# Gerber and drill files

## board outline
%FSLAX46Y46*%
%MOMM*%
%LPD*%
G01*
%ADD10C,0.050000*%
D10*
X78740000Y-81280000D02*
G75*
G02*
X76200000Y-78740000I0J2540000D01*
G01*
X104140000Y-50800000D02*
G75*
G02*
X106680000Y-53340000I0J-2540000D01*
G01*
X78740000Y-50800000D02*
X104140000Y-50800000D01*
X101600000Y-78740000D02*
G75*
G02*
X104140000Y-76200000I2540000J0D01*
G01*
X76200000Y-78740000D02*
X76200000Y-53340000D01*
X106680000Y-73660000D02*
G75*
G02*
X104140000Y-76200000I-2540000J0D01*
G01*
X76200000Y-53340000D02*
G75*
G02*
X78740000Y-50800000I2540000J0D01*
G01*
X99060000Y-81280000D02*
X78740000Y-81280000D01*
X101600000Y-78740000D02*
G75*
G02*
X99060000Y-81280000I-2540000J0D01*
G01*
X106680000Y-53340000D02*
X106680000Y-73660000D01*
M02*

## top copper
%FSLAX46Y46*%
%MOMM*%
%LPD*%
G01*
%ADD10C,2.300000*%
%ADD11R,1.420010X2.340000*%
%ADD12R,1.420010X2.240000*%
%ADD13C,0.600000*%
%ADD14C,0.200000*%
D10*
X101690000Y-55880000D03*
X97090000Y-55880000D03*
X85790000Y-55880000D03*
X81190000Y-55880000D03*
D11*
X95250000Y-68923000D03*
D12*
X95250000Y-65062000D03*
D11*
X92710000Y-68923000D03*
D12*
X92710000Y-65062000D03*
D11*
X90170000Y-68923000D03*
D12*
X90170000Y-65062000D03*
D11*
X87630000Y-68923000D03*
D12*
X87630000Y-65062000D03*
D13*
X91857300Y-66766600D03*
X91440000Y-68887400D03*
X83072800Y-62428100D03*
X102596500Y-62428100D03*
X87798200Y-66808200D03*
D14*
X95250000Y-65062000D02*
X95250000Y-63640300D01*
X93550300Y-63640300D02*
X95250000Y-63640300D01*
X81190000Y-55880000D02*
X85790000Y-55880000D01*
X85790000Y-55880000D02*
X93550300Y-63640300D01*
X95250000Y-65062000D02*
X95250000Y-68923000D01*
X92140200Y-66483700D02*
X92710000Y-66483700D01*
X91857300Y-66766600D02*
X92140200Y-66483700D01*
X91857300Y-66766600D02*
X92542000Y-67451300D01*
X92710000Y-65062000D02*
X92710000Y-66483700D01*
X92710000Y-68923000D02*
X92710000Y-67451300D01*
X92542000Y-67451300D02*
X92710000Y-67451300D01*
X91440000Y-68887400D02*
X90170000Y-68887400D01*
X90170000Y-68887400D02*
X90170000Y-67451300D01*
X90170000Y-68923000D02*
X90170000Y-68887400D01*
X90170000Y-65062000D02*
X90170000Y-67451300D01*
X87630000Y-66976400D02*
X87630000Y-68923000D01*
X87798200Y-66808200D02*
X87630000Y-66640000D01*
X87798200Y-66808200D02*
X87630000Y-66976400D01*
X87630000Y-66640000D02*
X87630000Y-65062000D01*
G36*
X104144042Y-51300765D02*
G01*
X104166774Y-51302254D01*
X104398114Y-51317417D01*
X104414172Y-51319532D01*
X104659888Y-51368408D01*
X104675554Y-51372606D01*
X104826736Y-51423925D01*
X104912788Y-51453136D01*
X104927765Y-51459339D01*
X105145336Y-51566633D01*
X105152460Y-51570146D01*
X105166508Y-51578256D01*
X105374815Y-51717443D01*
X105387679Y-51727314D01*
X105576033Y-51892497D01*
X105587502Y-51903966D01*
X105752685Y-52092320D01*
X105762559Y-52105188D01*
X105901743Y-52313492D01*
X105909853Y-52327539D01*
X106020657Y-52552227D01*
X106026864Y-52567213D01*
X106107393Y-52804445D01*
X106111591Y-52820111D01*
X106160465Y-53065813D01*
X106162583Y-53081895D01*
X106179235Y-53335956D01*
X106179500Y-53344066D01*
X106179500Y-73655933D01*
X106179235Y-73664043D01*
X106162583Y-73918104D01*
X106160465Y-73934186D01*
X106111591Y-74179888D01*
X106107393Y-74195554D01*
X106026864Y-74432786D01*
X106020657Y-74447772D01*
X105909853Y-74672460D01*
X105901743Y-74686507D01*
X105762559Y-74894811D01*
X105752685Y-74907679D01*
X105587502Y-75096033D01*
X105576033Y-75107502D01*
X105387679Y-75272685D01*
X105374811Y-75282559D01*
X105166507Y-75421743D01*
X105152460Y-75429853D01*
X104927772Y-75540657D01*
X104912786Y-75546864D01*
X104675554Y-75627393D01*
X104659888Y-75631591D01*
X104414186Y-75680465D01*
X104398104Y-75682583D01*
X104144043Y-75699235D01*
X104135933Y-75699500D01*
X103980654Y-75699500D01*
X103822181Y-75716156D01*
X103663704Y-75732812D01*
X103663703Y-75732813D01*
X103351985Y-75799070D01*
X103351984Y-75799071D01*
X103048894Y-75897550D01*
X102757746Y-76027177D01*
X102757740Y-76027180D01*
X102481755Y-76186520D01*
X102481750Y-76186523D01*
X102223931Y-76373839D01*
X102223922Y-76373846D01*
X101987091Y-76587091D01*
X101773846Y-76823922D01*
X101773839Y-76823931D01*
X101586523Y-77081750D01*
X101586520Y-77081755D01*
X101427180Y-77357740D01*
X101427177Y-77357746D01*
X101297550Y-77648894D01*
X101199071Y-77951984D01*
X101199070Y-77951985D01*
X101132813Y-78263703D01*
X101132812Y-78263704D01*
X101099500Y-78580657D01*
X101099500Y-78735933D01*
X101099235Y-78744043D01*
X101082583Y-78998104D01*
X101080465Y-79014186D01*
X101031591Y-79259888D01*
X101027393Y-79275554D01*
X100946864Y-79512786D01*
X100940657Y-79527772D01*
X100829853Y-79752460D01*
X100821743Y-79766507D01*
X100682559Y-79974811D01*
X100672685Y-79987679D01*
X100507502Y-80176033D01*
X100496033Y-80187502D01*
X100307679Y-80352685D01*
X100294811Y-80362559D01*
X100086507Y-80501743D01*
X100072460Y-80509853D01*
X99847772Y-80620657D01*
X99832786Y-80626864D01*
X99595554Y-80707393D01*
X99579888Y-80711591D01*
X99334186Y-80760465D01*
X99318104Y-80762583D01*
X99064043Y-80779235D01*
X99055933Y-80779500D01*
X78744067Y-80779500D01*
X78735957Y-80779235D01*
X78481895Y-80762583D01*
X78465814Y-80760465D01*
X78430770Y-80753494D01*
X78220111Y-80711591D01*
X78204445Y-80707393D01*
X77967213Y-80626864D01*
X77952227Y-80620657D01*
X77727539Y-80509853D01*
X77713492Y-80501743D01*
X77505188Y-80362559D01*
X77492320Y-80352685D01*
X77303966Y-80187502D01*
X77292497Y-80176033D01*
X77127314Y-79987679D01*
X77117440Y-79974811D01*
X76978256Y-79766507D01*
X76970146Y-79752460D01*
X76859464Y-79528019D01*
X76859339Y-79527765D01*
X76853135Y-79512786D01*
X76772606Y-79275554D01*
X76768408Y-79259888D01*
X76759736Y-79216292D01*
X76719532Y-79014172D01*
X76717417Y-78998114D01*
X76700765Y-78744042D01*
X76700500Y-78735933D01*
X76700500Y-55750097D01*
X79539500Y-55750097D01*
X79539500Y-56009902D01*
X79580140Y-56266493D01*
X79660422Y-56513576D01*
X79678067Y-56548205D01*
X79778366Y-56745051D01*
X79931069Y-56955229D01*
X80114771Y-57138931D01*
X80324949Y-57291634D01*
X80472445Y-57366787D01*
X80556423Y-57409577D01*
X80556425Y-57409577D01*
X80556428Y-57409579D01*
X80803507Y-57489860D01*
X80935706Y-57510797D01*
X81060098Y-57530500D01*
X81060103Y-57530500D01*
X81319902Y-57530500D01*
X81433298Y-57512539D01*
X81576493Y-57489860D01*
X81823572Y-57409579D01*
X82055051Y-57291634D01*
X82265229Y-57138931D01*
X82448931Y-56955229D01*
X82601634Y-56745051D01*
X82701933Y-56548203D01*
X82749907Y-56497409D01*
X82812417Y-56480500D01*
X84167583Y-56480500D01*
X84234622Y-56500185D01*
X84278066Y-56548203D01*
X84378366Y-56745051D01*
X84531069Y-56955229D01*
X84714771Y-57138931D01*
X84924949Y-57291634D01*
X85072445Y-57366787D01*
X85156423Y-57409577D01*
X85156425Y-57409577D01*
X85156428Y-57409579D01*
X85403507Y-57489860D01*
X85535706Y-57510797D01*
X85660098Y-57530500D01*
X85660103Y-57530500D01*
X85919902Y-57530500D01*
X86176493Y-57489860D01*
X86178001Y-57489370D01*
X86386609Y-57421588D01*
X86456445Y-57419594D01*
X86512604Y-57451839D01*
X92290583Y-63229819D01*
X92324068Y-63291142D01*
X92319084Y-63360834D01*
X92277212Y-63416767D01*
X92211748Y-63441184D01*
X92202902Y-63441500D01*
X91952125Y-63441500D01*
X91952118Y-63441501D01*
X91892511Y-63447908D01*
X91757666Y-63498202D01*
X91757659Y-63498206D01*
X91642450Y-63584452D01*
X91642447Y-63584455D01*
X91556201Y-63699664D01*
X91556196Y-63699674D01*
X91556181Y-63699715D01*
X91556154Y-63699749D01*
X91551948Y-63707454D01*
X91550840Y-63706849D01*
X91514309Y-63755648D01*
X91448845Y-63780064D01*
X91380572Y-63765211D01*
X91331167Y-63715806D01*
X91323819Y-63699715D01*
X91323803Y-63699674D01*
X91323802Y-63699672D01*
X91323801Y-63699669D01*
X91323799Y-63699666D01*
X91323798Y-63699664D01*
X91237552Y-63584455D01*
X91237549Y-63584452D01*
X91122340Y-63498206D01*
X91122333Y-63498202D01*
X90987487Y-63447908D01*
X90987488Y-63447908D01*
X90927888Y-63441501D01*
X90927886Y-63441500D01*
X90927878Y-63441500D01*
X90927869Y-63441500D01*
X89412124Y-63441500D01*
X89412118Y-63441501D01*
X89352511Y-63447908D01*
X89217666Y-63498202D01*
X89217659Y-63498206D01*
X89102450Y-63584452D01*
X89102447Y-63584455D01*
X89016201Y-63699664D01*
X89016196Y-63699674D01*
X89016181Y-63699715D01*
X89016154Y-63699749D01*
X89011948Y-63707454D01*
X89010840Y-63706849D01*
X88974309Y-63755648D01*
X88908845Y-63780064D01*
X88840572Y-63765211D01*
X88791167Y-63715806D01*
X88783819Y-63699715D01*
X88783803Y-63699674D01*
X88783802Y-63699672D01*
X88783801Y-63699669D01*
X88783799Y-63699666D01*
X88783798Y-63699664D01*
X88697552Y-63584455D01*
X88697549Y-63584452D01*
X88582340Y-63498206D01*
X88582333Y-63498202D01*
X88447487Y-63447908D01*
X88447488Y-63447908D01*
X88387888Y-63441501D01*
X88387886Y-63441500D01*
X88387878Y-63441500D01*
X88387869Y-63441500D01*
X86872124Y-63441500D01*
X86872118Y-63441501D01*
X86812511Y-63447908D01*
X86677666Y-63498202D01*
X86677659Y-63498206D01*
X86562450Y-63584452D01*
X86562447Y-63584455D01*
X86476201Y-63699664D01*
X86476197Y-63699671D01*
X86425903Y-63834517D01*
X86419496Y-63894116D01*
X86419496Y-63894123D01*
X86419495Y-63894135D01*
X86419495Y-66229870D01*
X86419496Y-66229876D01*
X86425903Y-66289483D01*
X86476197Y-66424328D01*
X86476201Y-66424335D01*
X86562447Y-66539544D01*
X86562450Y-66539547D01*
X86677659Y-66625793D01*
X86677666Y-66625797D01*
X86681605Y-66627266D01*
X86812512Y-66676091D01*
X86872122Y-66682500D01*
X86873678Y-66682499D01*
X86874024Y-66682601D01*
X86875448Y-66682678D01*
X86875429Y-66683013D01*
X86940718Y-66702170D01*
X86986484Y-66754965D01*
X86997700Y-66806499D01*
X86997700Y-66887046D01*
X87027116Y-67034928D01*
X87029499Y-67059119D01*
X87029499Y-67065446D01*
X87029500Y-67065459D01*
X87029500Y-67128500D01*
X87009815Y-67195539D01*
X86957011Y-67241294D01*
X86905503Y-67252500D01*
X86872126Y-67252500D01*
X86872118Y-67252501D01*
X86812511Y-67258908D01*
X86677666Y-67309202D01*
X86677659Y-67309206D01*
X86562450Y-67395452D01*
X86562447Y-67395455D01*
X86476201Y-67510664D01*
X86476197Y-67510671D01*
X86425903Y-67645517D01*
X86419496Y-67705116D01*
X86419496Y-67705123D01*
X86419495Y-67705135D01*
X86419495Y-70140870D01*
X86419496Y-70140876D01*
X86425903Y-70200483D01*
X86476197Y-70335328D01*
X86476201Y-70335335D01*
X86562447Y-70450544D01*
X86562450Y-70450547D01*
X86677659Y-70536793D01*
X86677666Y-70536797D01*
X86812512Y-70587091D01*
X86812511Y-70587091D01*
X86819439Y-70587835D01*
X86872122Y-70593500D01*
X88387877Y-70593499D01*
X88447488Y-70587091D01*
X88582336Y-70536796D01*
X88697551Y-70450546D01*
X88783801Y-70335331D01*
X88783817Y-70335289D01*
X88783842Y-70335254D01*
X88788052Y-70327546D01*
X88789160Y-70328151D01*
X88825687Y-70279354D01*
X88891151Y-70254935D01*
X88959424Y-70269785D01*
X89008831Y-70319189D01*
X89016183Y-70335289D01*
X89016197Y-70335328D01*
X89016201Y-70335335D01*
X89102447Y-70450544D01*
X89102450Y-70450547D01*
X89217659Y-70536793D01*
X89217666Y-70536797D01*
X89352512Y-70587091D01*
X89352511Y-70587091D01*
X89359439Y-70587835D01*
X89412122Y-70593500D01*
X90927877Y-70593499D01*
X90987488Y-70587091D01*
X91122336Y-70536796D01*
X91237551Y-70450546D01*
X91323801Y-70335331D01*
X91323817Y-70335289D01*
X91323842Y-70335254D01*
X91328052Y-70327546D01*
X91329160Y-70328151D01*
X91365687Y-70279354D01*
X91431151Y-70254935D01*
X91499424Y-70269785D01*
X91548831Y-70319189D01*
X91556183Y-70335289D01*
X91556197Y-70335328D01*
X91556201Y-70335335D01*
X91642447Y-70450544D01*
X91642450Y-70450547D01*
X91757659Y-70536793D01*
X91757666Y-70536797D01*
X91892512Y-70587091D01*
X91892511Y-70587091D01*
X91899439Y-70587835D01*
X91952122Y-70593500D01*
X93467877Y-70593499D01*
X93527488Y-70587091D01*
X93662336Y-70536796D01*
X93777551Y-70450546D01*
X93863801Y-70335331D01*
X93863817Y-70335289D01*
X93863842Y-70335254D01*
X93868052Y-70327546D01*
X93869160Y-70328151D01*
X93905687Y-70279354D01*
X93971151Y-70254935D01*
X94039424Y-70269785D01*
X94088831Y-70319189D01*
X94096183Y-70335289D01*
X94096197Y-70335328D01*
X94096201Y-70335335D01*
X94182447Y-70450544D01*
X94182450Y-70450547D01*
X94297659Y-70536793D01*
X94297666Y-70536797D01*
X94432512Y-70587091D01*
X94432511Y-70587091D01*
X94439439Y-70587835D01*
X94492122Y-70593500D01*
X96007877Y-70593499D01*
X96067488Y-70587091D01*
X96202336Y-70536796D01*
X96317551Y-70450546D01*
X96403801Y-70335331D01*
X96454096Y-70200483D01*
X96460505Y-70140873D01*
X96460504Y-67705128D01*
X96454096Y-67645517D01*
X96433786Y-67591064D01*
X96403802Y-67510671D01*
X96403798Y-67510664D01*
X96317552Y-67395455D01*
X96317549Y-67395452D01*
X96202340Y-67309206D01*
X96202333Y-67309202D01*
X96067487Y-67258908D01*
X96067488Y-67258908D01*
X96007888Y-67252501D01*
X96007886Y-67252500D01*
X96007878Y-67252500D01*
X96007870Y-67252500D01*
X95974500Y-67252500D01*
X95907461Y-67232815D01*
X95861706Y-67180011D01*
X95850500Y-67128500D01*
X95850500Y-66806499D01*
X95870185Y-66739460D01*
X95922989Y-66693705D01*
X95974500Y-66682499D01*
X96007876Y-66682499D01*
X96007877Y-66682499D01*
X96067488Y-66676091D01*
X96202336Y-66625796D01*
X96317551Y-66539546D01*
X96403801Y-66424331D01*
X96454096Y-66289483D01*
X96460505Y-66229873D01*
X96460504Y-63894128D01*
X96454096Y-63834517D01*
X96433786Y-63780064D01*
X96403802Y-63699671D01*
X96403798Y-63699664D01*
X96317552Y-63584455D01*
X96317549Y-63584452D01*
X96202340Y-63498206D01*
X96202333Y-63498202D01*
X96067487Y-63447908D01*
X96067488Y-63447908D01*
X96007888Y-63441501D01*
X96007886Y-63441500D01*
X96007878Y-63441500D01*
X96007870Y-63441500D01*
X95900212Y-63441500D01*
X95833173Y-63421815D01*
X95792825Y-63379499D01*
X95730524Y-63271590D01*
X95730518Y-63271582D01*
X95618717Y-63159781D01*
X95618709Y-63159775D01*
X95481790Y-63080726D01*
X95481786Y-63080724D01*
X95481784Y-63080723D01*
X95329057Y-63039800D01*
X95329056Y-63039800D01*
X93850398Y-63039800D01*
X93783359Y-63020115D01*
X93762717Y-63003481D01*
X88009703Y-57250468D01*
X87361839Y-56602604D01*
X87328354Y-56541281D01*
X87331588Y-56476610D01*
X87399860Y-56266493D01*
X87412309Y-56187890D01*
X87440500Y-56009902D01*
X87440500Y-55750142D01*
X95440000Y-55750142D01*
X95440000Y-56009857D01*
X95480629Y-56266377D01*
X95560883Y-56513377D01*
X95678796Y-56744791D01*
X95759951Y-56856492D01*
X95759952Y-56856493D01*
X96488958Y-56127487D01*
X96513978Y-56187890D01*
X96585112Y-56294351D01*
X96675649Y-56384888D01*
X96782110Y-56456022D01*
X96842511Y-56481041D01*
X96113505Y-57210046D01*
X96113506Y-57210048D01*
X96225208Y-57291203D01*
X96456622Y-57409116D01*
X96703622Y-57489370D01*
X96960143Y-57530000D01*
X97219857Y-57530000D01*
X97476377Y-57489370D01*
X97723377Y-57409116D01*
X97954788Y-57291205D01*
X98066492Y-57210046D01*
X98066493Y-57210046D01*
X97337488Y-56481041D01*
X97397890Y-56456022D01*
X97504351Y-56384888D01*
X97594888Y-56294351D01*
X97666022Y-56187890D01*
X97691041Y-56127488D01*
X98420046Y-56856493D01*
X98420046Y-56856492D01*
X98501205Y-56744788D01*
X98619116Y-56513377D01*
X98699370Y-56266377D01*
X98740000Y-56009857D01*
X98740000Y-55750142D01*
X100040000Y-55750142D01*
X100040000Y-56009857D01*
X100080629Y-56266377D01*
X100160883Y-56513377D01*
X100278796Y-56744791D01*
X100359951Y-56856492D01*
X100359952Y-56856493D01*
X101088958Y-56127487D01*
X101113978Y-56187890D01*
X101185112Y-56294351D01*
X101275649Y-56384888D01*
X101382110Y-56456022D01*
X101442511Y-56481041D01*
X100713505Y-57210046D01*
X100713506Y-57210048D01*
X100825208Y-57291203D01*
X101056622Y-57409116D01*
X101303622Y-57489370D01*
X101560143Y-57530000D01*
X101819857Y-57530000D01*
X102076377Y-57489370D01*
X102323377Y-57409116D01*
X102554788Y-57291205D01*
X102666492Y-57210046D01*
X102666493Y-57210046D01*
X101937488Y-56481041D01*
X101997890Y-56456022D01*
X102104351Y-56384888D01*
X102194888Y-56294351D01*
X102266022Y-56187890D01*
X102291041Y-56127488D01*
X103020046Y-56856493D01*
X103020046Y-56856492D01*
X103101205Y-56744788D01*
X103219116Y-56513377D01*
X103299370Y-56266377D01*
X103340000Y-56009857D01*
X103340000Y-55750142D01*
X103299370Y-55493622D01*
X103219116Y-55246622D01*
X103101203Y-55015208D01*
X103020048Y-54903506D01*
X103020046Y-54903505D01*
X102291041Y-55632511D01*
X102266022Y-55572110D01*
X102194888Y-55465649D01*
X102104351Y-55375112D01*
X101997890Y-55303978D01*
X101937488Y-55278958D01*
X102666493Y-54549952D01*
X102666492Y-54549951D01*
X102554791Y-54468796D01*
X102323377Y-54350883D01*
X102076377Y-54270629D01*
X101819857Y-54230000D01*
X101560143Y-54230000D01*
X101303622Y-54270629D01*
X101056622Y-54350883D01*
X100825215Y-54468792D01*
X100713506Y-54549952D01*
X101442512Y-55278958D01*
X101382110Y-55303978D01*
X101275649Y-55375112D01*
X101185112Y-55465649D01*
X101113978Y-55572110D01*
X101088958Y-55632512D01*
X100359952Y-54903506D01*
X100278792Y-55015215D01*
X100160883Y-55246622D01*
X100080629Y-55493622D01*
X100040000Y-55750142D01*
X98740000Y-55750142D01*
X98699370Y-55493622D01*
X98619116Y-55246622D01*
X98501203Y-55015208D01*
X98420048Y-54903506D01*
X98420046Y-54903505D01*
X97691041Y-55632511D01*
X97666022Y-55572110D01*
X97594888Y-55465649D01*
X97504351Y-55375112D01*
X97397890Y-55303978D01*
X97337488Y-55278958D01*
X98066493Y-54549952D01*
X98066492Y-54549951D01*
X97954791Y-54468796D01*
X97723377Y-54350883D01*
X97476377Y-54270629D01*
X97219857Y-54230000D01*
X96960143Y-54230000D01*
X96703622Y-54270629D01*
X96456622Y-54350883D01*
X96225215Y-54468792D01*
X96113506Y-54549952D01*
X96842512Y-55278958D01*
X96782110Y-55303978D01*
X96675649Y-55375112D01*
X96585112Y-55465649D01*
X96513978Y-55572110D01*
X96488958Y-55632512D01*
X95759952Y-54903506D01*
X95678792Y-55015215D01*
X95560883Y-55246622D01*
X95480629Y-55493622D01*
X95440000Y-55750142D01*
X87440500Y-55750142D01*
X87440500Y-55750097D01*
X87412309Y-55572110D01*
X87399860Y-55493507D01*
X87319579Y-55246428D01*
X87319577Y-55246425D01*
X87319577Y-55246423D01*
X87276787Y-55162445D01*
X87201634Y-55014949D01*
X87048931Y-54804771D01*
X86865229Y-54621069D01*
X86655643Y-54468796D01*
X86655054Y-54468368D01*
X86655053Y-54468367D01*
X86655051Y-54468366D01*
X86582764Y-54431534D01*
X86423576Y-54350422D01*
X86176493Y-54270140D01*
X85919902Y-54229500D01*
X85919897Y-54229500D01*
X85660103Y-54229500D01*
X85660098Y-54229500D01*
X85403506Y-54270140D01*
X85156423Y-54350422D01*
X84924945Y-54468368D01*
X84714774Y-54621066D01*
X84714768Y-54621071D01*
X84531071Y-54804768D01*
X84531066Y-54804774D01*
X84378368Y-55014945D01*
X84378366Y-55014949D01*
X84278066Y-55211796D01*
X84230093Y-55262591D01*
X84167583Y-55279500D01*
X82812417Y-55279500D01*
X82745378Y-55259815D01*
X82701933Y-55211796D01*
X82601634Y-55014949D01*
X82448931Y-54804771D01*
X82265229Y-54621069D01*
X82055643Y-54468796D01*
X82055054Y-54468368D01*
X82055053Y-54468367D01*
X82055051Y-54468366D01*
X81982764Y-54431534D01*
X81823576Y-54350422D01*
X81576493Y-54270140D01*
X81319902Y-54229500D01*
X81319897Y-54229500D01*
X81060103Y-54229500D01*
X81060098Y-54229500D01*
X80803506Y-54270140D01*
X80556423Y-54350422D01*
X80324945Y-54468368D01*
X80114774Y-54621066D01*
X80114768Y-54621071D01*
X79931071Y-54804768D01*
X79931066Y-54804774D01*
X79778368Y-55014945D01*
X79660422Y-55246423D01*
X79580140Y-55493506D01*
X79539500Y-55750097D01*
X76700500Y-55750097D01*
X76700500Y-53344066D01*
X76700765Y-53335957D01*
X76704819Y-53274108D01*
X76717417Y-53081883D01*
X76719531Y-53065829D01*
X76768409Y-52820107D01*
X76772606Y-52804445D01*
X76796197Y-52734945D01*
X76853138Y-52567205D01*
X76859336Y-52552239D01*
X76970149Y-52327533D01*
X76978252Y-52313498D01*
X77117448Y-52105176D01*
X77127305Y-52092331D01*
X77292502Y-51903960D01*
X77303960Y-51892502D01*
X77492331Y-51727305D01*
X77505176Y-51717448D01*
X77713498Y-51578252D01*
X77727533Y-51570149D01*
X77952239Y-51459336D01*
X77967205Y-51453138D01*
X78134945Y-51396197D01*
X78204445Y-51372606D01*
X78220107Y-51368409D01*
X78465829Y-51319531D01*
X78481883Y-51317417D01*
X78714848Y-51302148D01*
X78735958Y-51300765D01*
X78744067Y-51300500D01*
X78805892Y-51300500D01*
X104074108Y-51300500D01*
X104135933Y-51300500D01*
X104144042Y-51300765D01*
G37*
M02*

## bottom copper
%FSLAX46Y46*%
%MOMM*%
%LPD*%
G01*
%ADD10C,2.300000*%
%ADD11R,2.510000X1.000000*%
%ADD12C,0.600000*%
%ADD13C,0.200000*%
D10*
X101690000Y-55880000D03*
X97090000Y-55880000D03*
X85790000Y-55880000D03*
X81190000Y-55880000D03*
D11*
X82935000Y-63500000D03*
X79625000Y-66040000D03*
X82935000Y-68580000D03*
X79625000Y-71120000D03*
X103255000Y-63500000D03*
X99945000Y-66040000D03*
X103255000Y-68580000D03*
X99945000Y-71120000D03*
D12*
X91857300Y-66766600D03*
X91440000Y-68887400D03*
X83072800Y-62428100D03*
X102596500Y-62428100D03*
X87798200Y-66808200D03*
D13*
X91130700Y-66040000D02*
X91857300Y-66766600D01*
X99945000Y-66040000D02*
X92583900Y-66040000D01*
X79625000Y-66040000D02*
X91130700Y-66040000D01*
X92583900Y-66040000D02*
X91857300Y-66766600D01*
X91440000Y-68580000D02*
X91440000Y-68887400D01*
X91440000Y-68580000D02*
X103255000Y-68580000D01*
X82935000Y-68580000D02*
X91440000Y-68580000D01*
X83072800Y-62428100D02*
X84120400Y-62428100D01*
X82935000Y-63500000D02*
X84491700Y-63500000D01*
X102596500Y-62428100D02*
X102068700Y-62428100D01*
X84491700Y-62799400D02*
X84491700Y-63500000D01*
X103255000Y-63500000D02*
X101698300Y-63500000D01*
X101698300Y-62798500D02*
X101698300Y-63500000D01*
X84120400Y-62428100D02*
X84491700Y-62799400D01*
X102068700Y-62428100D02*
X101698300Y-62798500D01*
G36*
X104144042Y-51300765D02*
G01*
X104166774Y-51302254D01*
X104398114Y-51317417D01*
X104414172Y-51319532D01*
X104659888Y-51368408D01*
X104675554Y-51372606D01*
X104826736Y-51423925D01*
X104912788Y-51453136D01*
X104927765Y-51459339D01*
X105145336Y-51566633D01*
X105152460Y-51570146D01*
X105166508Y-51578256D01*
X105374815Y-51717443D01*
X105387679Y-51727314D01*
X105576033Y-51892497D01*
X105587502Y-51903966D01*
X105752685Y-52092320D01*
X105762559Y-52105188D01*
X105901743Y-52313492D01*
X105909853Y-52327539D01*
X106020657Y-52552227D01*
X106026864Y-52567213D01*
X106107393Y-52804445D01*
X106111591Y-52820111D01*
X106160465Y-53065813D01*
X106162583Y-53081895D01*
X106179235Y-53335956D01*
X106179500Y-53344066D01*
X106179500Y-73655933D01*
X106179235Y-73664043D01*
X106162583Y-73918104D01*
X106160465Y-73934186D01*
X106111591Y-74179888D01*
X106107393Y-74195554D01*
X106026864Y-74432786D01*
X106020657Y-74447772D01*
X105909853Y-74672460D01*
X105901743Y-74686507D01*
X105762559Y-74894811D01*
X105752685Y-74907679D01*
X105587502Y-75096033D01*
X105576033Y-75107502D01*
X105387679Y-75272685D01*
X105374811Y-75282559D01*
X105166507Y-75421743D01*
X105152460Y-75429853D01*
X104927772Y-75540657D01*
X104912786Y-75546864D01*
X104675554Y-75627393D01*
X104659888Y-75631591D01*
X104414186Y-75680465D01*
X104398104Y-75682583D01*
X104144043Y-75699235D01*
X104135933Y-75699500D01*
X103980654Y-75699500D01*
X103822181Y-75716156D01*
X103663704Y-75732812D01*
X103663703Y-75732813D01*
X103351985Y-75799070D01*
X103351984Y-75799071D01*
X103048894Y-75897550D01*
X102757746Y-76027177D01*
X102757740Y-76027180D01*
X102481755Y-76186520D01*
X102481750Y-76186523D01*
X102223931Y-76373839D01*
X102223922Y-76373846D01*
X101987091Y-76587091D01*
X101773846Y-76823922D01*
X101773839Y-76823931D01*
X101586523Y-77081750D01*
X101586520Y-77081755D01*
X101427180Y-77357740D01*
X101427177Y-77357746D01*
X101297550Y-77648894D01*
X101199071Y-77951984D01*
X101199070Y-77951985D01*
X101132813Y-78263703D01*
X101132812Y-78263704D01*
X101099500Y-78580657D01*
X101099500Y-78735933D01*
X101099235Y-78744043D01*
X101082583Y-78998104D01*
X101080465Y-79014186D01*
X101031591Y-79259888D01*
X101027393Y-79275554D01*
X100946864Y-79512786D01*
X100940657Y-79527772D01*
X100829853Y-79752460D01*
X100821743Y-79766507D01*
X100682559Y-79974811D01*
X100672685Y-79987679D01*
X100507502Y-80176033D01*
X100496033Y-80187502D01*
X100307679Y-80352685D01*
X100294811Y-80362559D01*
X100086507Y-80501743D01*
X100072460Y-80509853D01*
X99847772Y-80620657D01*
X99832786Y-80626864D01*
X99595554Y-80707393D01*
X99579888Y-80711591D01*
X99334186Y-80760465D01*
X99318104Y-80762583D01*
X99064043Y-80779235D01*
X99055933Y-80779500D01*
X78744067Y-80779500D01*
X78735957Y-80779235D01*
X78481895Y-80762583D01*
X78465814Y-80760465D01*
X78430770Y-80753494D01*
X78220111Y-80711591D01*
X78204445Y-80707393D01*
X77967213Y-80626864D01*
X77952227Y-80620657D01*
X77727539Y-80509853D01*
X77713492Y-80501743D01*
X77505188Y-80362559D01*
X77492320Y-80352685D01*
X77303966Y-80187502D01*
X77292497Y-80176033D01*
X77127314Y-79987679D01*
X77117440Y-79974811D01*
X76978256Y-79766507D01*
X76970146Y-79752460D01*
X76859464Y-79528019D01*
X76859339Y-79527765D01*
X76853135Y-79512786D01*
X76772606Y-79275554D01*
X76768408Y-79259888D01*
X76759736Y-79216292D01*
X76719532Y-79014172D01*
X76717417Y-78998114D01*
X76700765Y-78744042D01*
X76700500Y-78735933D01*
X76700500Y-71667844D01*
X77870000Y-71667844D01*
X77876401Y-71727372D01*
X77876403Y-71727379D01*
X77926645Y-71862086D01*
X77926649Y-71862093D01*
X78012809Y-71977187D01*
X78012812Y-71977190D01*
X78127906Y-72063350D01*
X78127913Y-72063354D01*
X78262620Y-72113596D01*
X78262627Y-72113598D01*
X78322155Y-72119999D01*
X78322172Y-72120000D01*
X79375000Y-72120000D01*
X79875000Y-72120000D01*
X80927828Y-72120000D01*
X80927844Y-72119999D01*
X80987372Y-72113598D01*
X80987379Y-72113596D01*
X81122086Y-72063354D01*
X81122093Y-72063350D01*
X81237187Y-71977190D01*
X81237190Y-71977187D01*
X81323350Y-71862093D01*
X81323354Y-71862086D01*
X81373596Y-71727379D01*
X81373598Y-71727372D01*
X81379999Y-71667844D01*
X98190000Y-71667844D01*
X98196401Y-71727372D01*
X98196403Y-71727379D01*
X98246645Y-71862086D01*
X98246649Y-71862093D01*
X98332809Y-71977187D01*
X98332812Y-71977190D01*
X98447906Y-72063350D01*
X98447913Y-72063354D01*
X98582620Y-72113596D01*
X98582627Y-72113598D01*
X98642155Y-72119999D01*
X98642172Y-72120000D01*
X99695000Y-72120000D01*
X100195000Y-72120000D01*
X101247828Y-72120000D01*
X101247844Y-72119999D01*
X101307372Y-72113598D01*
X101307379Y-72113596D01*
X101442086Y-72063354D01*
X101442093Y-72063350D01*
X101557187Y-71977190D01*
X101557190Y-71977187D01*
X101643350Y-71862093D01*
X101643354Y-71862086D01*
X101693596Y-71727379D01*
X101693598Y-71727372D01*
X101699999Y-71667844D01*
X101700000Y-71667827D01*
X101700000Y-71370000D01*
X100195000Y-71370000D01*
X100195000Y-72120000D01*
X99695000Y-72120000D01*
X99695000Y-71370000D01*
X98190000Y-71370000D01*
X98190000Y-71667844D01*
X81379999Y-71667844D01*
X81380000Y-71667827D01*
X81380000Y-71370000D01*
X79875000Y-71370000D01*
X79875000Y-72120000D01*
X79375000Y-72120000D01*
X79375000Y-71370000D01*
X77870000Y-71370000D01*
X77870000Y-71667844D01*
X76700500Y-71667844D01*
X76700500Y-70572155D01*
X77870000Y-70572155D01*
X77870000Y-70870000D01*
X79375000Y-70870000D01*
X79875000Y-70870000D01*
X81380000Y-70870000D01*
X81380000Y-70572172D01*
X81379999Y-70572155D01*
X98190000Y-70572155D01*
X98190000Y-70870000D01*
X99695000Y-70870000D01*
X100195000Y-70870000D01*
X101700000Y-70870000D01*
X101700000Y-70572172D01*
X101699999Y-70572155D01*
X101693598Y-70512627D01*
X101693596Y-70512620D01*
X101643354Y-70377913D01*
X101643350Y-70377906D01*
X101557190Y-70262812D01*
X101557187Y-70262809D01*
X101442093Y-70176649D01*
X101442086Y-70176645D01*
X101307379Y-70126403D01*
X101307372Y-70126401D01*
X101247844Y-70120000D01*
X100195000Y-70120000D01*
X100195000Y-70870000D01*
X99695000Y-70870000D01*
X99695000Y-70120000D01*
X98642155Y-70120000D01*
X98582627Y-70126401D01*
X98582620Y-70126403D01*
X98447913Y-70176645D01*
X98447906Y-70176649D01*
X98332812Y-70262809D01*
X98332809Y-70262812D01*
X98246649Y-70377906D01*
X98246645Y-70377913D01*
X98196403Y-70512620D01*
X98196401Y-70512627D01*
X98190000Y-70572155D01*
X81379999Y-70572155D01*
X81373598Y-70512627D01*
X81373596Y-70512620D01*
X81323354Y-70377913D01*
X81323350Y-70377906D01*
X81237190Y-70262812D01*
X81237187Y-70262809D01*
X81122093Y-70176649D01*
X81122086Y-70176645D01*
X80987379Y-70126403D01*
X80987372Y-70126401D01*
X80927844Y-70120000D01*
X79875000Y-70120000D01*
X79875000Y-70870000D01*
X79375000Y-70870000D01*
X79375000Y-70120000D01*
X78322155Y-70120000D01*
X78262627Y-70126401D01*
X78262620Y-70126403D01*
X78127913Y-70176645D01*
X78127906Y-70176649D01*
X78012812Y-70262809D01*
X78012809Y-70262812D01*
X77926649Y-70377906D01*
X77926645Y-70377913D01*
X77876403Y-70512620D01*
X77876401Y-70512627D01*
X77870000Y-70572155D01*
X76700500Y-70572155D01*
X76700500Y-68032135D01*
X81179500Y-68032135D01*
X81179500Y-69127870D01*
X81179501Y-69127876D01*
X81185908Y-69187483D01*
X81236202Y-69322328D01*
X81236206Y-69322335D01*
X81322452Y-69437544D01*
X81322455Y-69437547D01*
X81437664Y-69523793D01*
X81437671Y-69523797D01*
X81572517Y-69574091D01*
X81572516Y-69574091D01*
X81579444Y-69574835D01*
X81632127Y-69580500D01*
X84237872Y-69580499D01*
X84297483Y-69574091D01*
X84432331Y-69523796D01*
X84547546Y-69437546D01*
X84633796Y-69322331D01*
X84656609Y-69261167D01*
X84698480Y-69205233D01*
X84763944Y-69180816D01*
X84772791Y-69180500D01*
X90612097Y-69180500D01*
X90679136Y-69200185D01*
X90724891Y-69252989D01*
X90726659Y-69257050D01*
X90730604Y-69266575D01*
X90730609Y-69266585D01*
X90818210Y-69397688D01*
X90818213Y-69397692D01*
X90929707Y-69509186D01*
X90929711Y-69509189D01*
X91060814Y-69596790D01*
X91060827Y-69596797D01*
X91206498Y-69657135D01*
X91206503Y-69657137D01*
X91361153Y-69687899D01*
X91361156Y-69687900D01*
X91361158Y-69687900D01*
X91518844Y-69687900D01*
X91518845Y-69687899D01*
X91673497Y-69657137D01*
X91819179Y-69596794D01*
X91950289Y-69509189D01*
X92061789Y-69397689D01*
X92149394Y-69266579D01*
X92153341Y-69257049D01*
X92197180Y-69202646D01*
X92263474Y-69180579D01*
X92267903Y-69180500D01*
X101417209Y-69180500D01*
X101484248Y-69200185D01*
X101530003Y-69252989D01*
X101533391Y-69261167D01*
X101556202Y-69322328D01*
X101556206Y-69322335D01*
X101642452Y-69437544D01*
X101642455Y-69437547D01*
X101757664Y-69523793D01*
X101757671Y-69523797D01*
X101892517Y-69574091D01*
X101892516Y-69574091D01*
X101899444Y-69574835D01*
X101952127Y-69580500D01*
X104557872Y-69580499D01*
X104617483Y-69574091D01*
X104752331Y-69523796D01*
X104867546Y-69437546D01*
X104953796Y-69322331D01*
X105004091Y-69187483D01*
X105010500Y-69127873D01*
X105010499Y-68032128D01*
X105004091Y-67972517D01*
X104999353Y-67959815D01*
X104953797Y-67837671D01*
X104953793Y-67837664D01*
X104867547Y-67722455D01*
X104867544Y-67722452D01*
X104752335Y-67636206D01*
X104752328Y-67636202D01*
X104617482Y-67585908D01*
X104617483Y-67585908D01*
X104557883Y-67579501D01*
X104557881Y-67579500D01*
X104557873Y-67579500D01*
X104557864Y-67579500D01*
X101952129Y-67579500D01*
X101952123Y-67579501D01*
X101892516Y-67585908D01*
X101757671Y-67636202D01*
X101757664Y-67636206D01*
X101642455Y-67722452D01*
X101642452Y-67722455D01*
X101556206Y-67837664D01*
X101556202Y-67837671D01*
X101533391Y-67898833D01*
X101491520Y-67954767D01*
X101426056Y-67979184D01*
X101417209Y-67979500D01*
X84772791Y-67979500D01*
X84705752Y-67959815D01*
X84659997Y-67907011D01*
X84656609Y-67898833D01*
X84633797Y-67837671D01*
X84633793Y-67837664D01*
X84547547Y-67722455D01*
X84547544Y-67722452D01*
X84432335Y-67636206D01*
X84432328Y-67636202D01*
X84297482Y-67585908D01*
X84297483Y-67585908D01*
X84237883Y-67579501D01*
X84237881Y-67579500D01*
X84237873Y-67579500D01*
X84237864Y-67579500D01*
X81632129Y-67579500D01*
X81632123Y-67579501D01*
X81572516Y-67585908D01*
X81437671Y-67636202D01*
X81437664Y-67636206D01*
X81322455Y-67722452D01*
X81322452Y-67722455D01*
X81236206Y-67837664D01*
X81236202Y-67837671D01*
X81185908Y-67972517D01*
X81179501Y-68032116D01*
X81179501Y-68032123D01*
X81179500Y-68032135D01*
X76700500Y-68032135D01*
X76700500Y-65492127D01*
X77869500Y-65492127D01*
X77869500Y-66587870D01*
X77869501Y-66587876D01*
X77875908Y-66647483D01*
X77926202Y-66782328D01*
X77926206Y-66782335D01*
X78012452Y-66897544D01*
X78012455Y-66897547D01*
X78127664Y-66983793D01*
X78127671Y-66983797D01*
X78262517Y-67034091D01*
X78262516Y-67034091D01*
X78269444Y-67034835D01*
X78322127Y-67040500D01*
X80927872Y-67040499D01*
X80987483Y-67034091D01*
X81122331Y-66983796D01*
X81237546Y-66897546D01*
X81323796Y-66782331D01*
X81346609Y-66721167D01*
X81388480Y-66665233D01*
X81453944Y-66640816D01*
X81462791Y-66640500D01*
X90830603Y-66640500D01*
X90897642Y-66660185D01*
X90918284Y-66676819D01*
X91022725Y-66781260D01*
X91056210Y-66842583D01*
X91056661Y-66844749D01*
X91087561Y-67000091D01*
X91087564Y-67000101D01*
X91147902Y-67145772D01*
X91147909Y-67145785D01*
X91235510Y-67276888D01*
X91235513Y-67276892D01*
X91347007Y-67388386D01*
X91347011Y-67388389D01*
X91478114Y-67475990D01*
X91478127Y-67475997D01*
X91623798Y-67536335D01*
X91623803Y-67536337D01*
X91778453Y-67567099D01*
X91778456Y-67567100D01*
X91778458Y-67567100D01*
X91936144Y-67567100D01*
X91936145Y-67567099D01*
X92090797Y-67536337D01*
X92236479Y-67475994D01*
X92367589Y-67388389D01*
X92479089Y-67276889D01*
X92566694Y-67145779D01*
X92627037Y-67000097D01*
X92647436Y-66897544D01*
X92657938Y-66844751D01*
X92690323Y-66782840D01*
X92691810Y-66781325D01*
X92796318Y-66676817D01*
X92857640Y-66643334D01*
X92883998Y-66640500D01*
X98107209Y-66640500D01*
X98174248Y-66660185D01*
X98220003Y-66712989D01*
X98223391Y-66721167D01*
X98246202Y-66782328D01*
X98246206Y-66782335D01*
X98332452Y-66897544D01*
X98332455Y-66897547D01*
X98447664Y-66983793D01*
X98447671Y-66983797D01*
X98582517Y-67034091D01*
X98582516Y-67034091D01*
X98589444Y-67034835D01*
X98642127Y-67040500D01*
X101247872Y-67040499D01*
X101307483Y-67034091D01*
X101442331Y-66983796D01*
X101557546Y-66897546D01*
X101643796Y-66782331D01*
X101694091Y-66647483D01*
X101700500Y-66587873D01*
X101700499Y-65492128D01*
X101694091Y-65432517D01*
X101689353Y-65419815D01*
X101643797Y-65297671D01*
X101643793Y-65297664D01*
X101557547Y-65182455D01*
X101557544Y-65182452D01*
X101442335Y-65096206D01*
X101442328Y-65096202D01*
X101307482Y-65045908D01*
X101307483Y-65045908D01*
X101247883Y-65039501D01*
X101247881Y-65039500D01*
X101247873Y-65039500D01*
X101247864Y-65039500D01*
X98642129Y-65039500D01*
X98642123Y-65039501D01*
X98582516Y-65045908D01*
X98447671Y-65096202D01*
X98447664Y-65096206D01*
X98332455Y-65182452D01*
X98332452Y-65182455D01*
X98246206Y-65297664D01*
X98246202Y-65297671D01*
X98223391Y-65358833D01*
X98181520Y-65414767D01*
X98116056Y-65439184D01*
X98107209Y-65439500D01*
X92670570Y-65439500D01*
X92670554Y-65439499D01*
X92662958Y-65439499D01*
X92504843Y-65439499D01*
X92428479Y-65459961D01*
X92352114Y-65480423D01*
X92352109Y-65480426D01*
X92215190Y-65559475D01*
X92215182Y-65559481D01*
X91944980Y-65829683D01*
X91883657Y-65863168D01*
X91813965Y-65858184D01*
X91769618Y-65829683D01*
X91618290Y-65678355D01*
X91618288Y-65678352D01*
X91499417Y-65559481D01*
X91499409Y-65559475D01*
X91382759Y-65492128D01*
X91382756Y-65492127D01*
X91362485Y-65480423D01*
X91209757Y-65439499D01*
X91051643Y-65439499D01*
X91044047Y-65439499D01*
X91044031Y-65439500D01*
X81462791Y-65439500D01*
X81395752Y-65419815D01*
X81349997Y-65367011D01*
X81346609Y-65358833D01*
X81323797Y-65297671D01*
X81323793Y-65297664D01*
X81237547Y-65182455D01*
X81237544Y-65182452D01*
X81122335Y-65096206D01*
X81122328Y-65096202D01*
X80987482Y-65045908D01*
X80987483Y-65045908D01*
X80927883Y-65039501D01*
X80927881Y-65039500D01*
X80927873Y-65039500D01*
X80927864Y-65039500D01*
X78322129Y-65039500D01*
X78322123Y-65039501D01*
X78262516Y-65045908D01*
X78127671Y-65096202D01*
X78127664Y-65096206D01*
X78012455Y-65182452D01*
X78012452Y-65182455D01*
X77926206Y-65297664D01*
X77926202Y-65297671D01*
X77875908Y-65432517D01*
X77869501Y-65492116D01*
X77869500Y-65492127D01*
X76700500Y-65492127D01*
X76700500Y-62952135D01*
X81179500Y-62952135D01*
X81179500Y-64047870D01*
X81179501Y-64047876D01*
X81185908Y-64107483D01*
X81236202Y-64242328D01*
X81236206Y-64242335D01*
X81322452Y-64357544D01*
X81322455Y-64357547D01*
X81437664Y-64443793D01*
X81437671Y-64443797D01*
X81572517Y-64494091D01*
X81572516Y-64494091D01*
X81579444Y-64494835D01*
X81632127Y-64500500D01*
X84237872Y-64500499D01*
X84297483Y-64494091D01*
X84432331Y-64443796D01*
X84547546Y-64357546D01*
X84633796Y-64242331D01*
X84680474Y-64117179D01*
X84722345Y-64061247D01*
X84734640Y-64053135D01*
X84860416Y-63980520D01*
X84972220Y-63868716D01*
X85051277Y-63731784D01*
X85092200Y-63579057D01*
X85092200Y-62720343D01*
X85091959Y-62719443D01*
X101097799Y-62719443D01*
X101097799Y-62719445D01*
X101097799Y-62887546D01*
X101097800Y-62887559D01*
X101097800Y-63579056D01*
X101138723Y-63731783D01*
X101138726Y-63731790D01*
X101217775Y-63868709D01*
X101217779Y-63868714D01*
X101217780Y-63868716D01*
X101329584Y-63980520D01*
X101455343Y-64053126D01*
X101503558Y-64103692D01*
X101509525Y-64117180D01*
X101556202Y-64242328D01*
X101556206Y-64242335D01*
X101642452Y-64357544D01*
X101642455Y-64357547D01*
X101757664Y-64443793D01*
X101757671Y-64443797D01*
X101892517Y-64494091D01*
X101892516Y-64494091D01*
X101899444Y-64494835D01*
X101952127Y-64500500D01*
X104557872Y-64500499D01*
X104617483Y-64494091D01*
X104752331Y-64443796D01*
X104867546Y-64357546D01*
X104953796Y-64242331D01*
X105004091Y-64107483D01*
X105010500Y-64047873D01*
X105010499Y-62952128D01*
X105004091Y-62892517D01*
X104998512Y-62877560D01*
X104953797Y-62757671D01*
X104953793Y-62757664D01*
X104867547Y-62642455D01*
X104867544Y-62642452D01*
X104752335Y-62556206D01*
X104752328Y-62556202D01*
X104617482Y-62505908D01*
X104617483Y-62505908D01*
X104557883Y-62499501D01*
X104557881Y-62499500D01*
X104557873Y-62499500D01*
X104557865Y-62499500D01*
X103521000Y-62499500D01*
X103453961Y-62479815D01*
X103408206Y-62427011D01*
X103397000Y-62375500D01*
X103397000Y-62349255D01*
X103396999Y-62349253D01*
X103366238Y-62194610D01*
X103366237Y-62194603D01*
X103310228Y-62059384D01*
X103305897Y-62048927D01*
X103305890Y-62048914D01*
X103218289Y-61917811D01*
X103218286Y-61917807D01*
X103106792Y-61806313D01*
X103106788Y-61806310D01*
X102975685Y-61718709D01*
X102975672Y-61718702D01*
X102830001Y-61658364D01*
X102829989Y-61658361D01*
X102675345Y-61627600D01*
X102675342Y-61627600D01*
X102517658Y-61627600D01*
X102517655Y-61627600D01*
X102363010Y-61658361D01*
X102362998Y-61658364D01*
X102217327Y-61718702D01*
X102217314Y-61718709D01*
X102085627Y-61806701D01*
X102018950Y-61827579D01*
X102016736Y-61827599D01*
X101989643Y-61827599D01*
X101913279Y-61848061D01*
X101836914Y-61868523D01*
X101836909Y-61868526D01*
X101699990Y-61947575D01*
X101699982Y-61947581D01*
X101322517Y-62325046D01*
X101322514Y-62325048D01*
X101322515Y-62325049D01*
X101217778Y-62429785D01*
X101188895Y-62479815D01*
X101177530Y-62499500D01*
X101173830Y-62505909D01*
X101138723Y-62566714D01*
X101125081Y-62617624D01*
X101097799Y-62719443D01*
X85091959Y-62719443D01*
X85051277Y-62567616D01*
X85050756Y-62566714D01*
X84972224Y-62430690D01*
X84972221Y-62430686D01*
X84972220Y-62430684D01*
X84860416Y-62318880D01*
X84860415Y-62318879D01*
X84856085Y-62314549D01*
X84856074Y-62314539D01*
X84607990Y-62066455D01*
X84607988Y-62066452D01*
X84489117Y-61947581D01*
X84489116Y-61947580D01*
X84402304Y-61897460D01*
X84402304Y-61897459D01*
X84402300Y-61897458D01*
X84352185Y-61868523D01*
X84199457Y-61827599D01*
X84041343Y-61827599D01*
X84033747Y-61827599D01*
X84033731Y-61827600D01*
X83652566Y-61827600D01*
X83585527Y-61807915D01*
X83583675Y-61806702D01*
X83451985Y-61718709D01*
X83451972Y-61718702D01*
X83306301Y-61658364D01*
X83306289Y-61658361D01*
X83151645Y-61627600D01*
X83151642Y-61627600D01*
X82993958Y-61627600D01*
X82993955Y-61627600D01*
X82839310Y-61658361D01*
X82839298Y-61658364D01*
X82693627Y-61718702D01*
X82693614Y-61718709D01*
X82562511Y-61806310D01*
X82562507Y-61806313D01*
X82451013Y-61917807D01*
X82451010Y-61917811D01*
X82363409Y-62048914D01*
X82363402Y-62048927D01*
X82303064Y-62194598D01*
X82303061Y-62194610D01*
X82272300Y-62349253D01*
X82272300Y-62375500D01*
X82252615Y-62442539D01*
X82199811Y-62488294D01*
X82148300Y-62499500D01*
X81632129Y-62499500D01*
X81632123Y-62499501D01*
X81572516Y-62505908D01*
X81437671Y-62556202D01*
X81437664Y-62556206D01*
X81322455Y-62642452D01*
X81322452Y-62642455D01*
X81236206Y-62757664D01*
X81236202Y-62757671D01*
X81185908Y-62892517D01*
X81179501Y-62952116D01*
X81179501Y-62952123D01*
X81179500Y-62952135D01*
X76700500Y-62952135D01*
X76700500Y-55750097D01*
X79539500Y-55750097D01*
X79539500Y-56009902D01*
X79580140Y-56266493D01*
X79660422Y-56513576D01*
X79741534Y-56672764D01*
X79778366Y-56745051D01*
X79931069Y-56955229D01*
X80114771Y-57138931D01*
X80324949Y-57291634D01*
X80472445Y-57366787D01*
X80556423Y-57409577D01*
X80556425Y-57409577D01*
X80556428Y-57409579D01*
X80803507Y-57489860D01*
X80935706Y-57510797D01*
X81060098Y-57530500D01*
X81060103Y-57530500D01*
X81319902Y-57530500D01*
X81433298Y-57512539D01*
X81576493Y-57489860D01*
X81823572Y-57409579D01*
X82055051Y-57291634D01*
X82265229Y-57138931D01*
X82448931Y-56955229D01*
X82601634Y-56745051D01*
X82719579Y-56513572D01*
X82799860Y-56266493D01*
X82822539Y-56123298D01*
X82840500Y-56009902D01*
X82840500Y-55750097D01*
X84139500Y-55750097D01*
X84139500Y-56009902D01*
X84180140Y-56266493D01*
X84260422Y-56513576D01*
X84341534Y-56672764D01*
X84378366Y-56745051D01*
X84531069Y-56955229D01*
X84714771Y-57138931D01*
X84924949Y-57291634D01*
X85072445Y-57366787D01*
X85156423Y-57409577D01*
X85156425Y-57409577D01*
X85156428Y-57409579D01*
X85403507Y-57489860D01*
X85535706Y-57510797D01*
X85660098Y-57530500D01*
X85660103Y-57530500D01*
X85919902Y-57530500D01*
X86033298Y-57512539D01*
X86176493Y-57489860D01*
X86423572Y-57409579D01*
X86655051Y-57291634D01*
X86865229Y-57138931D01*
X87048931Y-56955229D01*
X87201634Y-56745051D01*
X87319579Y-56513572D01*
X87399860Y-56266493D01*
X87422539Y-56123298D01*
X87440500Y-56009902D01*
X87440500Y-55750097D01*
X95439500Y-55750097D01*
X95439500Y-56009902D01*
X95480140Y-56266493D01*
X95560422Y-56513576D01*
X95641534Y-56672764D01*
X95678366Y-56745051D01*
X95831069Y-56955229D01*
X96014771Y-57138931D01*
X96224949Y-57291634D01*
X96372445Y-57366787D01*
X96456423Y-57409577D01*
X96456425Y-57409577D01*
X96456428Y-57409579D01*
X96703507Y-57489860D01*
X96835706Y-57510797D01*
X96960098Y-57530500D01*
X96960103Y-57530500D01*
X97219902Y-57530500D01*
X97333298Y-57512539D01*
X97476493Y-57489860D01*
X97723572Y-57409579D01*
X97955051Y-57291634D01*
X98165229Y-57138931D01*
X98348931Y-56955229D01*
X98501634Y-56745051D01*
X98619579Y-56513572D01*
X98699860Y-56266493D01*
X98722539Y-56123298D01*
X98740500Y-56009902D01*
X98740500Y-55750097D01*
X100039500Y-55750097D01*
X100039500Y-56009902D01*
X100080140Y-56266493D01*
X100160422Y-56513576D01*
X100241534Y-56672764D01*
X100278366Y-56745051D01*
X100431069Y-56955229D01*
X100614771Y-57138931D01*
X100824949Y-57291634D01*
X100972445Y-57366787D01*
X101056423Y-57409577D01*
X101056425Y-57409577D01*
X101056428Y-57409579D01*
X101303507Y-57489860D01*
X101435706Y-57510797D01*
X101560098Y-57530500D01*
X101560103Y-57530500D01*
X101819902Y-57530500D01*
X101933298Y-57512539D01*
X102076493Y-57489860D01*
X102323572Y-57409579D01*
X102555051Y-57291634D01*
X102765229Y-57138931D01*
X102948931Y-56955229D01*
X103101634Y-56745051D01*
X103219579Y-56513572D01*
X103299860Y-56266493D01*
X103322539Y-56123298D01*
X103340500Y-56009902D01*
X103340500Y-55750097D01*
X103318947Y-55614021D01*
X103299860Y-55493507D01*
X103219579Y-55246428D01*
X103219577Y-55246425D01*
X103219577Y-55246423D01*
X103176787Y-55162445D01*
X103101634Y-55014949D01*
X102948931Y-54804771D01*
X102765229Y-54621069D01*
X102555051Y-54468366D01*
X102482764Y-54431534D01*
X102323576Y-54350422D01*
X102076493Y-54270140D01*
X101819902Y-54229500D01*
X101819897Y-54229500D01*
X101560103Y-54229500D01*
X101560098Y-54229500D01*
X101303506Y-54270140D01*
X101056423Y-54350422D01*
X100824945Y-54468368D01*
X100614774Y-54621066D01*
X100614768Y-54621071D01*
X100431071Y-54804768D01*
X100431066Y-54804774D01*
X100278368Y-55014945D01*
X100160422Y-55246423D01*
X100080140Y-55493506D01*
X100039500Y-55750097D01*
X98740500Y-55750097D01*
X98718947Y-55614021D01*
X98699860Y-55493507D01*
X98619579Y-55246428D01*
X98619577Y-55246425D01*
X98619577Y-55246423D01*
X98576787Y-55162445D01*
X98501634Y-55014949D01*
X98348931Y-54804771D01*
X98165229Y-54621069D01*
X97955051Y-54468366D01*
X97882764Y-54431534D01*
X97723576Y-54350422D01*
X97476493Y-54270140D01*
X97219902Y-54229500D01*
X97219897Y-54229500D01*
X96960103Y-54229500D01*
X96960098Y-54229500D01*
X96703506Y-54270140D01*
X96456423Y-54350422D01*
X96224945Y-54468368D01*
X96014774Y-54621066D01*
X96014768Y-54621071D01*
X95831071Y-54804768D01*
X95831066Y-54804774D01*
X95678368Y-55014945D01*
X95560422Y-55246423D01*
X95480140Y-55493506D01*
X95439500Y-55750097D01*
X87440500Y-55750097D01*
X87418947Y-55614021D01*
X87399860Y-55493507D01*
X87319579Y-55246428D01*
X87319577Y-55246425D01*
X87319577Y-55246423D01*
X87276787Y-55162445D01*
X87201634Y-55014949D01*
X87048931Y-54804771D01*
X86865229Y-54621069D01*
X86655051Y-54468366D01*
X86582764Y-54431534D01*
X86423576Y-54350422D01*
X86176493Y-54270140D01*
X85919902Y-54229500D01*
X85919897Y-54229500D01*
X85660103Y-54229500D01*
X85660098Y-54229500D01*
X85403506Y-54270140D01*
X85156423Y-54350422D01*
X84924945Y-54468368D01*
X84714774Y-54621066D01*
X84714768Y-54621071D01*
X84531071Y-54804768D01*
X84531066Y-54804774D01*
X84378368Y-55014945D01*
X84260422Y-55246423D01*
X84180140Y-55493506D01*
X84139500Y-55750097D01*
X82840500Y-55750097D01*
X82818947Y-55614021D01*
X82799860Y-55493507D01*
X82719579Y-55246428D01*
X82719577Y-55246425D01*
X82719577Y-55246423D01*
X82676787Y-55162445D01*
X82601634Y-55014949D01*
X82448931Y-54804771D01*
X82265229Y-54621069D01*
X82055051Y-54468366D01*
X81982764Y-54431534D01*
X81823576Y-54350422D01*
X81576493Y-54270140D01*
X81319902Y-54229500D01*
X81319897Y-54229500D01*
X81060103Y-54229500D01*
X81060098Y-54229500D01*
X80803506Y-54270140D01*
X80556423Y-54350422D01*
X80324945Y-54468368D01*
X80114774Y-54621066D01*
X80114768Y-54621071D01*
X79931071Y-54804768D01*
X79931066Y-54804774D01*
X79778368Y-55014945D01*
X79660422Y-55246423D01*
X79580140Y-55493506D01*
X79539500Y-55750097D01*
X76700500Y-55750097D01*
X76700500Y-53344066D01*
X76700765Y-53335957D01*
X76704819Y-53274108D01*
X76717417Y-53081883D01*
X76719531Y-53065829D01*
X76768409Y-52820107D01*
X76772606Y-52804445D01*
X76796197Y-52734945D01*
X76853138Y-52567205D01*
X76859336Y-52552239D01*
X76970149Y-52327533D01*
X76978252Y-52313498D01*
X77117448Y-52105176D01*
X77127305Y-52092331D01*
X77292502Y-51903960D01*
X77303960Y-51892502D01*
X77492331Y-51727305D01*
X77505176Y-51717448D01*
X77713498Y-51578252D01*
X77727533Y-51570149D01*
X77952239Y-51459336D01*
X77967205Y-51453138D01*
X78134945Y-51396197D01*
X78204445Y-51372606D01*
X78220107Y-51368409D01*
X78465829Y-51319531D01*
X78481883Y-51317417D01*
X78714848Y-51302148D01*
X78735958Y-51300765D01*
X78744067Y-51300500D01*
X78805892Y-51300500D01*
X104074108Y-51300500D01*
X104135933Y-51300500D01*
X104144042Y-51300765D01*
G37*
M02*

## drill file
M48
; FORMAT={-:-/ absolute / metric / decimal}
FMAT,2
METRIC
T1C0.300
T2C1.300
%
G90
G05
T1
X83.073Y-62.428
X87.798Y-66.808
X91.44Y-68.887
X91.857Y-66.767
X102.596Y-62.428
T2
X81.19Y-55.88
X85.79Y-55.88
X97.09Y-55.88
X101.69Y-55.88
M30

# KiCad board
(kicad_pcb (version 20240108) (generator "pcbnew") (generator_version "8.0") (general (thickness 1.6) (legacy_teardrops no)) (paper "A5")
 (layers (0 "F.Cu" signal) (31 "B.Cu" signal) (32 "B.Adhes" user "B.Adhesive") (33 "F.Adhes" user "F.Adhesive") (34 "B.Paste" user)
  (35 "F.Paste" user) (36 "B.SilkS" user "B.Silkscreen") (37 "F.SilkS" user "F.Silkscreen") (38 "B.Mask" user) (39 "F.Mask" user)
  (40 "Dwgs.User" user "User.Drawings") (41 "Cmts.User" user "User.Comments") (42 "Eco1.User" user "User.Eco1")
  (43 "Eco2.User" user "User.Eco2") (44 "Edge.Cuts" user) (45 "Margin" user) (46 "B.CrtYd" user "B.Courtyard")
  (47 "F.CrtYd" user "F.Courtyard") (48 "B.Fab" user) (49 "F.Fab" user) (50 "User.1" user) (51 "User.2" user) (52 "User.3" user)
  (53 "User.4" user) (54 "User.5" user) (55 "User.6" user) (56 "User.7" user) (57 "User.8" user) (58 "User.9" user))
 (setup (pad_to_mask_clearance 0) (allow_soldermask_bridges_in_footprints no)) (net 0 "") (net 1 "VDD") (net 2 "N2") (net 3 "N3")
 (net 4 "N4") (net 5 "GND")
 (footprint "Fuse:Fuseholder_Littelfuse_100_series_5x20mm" (layer "F.Cu") (at 101.69 55.88 180)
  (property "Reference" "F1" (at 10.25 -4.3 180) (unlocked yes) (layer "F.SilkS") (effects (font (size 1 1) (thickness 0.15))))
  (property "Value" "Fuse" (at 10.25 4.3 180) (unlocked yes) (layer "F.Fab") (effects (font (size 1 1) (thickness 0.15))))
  (pad "1" thru_hole circle (at 0 0 180) (size 2.3 2.3) (drill 1.3) (layers "*.Cu" "*.Mask") (remove_unused_layers no) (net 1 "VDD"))
  (pad "1" thru_hole circle (at 4.6 0 180) (size 2.3 2.3) (drill 1.3) (layers "*.Cu" "*.Mask") (remove_unused_layers no) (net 1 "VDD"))
  (pad "2" thru_hole circle (at 15.9 0 180) (size 2.3 2.3) (drill 1.3) (layers "*.Cu" "*.Mask") (remove_unused_layers no) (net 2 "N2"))
  (pad "2" thru_hole circle (at 20.5 0 180) (size 2.3 2.3) (drill 1.3) (layers "*.Cu" "*.Mask") (remove_unused_layers no) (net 2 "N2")))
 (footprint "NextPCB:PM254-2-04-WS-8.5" (layer "F.Cu") (at 91.44 76.2 180)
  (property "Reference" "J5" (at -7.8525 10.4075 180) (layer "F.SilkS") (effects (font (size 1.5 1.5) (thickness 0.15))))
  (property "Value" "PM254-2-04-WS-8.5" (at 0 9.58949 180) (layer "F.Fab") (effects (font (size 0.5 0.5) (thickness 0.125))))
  (pad "1" smd rect (at -3.81 7.277 180) (size 1.42001 2.34) (layers "F.Cu" "F.Paste") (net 2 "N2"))
  (pad "2" smd rect (at -3.81 11.138 180) (size 1.42001 2.24) (layers "F.Cu" "F.Paste") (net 2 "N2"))
  (pad "3" smd rect (at -1.27 7.277 180) (size 1.42001 2.34) (layers "F.Cu" "F.Paste") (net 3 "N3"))
  (pad "4" smd rect (at -1.27 11.138 180) (size 1.42001 2.24) (layers "F.Cu" "F.Paste") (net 3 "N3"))
  (pad "5" smd rect (at 1.27 7.277 180) (size 1.42001 2.34) (layers "F.Cu" "F.Paste") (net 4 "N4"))
  (pad "6" smd rect (at 1.27 11.138 180) (size 1.42001 2.24) (layers "F.Cu" "F.Paste") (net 4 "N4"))
  (pad "7" smd rect (at 3.81 7.277 180) (size 1.42001 2.34) (layers "F.Cu" "F.Paste") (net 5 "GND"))
  (pad "8" smd rect (at 3.81 11.138 180) (size 1.42001 2.24) (layers "F.Cu" "F.Paste") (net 5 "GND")))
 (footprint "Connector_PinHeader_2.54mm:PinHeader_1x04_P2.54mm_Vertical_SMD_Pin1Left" (layer "B.Cu") (at 81.28 67.31 180)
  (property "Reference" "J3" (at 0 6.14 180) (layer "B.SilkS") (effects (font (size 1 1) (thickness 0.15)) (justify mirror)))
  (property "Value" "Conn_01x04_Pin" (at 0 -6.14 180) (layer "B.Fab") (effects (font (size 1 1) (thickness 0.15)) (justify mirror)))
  (pad "1" smd rect (at -1.655 3.81 180) (size 2.51 1) (layers "B.Cu" "B.Paste" "B.Mask") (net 1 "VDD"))
  (pad "2" smd rect (at 1.655 1.27 180) (size 2.51 1) (layers "B.Cu" "B.Paste" "B.Mask") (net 3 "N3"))
  (pad "3" smd rect (at -1.655 -1.27 180) (size 2.51 1) (layers "B.Cu" "B.Paste" "B.Mask") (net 4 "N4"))
  (pad "4" smd rect (at 1.655 -3.81 180) (size 2.51 1) (layers "B.Cu" "B.Paste" "B.Mask") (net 5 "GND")))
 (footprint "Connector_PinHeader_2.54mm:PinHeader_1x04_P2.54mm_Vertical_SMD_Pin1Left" (layer "B.Cu") (at 101.6 67.31 180)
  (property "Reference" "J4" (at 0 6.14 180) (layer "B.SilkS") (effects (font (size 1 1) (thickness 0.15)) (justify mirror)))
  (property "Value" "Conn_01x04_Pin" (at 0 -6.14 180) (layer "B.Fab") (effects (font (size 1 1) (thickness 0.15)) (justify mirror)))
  (pad "1" smd rect (at -1.655 3.81 180) (size 2.51 1) (layers "B.Cu" "B.Paste" "B.Mask") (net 1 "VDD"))
  (pad "2" smd rect (at 1.655 1.27 180) (size 2.51 1) (layers "B.Cu" "B.Paste" "B.Mask") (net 3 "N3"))
  (pad "3" smd rect (at -1.655 -1.27 180) (size 2.51 1) (layers "B.Cu" "B.Paste" "B.Mask") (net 4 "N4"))
  (pad "4" smd rect (at 1.655 -3.81 180) (size 2.51 1) (layers "B.Cu" "B.Paste" "B.Mask") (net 5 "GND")))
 (gr_arc (start 78.74 81.28) (mid 76.943949 80.536051) (end 76.2 78.74) (stroke (width 0.05) (type default)) (layer "Edge.Cuts"))
 (gr_arc (start 104.14 50.8) (mid 105.936051 51.543949) (end 106.68 53.34) (stroke (width 0.05) (type default)) (layer "Edge.Cuts"))
 (gr_line (start 78.74 50.8) (end 104.14 50.8) (stroke (width 0.05) (type default)) (layer "Edge.Cuts"))
 (gr_arc (start 101.6 78.74) (mid 102.343949 76.943949) (end 104.14 76.2) (stroke (width 0.05) (type default)) (layer "Edge.Cuts"))
 (gr_line (start 76.2 78.74) (end 76.2 53.34) (stroke (width 0.05) (type default)) (layer "Edge.Cuts"))
 (gr_arc (start 106.68 73.66) (mid 105.936051 75.456051) (end 104.14 76.2) (stroke (width 0.05) (type default)) (layer "Edge.Cuts"))
 (gr_arc (start 76.2 53.34) (mid 76.943949 51.543949) (end 78.74 50.8) (stroke (width 0.05) (type default)) (layer "Edge.Cuts"))
 (gr_line (start 99.06 81.28) (end 78.74 81.28) (stroke (width 0.05) (type default)) (layer "Edge.Cuts"))
 (gr_arc (start 101.6 78.74) (mid 100.856051 80.536051) (end 99.06 81.28) (stroke (width 0.05) (type default)) (layer "Edge.Cuts"))
 (gr_line (start 106.68 53.34) (end 106.68 73.66) (stroke (width 0.05) (type default)) (layer "Edge.Cuts"))
 (segment (start 95.25 65.062) (end 95.25 63.6403) (width 0.2) (layer "F.Cu") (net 2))
 (segment (start 93.5503 63.6403) (end 95.25 63.6403) (width 0.2) (layer "F.Cu") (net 2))
 (segment (start 81.19 55.88) (end 85.79 55.88) (width 0.2) (layer "F.Cu") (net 2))
 (segment (start 85.79 55.88) (end 93.5503 63.6403) (width 0.2) (layer "F.Cu") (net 2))
 (segment (start 95.25 65.062) (end 95.25 68.923) (width 0.2) (layer "F.Cu") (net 2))
 (segment (start 92.1402 66.4837) (end 92.71 66.4837) (width 0.2) (layer "F.Cu") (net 3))
 (segment (start 91.8573 66.7666) (end 92.1402 66.4837) (width 0.2) (layer "F.Cu") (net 3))
 (segment (start 91.8573 66.7666) (end 92.542 67.4513) (width 0.2) (layer "F.Cu") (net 3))
 (segment (start 92.71 65.062) (end 92.71 66.4837) (width 0.2) (layer "F.Cu") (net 3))
 (segment (start 92.71 68.923) (end 92.71 67.4513) (width 0.2) (layer "F.Cu") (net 3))
 (segment (start 92.542 67.4513) (end 92.71 67.4513) (width 0.2) (layer "F.Cu") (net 3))
 (via (at 91.8573 66.7666) (size 0.6) (drill 0.3) (layers "F.Cu" "B.Cu") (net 3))
 (segment (start 91.1307 66.04) (end 91.8573 66.7666) (width 0.2) (layer "B.Cu") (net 3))
 (segment (start 99.945 66.04) (end 92.5839 66.04) (width 0.2) (layer "B.Cu") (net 3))
 (segment (start 79.625 66.04) (end 91.1307 66.04) (width 0.2) (layer "B.Cu") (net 3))
 (segment (start 92.5839 66.04) (end 91.8573 66.7666) (width 0.2) (layer "B.Cu") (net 3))
 (segment (start 91.44 68.8874) (end 90.17 68.8874) (width 0.2) (layer "F.Cu") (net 4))
 (segment (start 90.17 68.8874) (end 90.17 67.4513) (width 0.2) (layer "F.Cu") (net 4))
 (segment (start 90.17 68.923) (end 90.17 68.8874) (width 0.2) (layer "F.Cu") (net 4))
 (segment (start 90.17 65.062) (end 90.17 67.4513) (width 0.2) (layer "F.Cu") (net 4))
 (via (at 91.44 68.8874) (size 0.6) (drill 0.3) (layers "F.Cu" "B.Cu") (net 4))
 (segment (start 91.44 68.58) (end 91.44 68.8874) (width 0.2) (layer "B.Cu") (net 4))
 (segment (start 91.44 68.58) (end 103.255 68.58) (width 0.2) (layer "B.Cu") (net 4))
 (segment (start 82.935 68.58) (end 91.44 68.58) (width 0.2) (layer "B.Cu") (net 4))
 (via (at 83.0728 62.4281) (size 0.6) (drill 0.3) (layers "F.Cu" "B.Cu") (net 1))
 (via (at 102.5965 62.4281) (size 0.6) (drill 0.3) (layers "F.Cu" "B.Cu") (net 1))
 (segment (start 83.0728 62.4281) (end 84.1204 62.4281) (width 0.2) (layer "B.Cu") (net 1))
 (segment (start 82.935 63.5) (end 84.4917 63.5) (width 0.2) (layer "B.Cu") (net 1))
 (segment (start 102.5965 62.4281) (end 102.0687 62.4281) (width 0.2) (layer "B.Cu") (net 1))
 (segment (start 84.4917 62.7994) (end 84.4917 63.5) (width 0.2) (layer "B.Cu") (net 1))
 (segment (start 103.255 63.5) (end 101.6983 63.5) (width 0.2) (layer "B.Cu") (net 1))
 (segment (start 101.6983 62.7985) (end 101.6983 63.5) (width 0.2) (layer "B.Cu") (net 1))
 (segment (start 84.1204 62.4281) (end 84.4917 62.7994) (width 0.2) (layer "B.Cu") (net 1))
 (segment (start 102.0687 62.4281) (end 101.6983 62.7985) (width 0.2) (layer "B.Cu") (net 1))
 (segment (start 87.63 66.9764) (end 87.63 68.923) (width 0.2) (layer "F.Cu") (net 5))
 (segment (start 87.7982 66.8082) (end 87.63 66.64) (width 0.2) (layer "F.Cu") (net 5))
 (segment (start 87.7982 66.8082) (end 87.63 66.9764) (width 0.2) (layer "F.Cu") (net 5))
 (segment (start 87.63 66.64) (end 87.63 65.062) (width 0.2) (layer "F.Cu") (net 5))
 (via (at 87.7982 66.8082) (size 0.6) (drill 0.3) (layers "F.Cu" "B.Cu") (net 5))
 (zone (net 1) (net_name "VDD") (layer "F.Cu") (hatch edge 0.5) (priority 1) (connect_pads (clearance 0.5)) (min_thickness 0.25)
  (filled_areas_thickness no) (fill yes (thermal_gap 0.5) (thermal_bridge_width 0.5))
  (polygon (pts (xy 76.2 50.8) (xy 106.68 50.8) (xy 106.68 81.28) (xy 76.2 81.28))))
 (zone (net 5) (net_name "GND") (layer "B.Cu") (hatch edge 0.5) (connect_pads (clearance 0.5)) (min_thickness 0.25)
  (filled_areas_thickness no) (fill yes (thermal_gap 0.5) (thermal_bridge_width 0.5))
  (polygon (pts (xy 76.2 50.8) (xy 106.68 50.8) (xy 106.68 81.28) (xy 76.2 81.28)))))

